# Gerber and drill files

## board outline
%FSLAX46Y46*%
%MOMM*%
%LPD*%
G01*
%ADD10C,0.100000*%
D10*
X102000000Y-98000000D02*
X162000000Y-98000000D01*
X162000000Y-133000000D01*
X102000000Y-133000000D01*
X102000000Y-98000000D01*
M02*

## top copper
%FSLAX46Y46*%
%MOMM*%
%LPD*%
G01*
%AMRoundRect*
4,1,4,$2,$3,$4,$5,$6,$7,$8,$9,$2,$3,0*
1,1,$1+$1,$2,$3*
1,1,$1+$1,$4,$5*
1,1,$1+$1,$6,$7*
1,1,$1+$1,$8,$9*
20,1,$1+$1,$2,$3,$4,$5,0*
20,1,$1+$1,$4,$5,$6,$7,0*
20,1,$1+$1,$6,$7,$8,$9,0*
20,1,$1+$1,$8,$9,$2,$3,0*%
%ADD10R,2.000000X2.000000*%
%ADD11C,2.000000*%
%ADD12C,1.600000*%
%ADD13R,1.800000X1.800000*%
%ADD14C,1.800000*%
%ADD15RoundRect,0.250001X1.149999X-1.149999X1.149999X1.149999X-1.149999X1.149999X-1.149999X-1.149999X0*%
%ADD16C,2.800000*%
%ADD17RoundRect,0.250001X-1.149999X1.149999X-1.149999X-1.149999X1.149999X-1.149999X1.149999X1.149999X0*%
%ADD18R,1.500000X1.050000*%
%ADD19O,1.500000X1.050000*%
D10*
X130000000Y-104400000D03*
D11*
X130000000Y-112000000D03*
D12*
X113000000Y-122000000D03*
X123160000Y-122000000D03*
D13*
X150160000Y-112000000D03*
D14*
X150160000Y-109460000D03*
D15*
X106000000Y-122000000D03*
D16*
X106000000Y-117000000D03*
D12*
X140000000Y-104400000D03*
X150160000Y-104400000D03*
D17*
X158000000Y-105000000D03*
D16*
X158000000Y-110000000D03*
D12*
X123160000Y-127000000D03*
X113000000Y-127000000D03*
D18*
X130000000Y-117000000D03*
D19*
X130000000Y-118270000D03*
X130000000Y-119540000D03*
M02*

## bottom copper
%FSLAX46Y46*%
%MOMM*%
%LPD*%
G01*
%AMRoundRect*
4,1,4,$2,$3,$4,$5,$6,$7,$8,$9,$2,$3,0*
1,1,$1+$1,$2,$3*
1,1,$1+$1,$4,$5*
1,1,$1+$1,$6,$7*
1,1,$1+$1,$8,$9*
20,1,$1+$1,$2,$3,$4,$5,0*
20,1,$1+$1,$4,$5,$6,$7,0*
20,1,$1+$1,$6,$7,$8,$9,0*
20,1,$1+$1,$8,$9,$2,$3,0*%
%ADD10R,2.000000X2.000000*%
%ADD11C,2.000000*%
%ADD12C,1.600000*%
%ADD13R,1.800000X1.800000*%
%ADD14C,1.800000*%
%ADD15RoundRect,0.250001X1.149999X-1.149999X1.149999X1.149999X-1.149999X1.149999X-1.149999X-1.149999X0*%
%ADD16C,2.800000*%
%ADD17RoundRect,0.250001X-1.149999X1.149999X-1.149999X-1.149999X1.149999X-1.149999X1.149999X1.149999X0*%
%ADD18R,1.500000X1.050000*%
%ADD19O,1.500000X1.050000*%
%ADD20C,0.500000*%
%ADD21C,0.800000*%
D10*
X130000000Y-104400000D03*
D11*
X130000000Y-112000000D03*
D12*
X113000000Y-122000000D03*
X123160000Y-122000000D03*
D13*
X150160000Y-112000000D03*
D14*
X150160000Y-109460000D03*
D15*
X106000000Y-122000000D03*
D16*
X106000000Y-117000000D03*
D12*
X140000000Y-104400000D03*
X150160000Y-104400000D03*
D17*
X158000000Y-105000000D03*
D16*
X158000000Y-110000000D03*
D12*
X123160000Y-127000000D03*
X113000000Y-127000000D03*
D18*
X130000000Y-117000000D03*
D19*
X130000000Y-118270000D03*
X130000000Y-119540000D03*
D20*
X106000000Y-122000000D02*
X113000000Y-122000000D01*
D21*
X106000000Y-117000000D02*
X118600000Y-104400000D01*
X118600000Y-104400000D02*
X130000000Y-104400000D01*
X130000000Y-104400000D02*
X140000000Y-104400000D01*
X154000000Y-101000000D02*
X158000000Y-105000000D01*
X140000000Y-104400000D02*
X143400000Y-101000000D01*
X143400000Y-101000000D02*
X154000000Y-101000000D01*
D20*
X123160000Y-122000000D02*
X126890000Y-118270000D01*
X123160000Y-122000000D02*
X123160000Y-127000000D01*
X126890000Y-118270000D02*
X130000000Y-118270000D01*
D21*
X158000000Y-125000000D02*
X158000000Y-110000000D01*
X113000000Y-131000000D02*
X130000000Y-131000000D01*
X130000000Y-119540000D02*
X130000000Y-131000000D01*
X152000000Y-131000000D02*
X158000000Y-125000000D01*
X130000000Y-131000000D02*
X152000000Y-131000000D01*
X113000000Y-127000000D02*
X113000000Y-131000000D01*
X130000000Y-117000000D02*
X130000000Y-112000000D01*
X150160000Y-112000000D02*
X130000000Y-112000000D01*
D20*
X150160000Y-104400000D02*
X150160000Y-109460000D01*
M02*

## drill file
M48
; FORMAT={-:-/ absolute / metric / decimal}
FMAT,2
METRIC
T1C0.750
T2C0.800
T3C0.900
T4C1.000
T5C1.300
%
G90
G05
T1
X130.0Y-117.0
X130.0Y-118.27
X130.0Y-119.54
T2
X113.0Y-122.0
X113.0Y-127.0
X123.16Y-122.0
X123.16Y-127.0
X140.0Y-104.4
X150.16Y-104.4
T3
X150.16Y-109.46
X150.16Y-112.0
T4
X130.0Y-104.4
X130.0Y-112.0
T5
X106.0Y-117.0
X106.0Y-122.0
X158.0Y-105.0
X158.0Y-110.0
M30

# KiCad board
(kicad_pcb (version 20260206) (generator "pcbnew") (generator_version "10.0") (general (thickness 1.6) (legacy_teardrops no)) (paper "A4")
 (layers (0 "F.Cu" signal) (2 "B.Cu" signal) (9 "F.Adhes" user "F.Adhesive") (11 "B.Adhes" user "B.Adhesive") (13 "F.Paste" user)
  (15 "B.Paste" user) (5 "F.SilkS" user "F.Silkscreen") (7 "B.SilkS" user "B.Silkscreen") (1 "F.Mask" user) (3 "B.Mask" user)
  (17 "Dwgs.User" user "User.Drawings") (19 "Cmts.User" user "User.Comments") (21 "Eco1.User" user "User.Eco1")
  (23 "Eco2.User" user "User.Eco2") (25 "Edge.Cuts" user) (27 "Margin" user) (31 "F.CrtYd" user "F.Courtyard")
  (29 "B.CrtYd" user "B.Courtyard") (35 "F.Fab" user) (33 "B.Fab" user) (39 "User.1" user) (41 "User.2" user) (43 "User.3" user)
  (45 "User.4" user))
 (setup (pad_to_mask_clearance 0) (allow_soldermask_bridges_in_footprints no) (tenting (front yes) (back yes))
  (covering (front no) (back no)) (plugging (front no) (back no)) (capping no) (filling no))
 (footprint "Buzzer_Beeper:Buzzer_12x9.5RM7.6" (layer "F.Cu") (at 130 104.4 -90)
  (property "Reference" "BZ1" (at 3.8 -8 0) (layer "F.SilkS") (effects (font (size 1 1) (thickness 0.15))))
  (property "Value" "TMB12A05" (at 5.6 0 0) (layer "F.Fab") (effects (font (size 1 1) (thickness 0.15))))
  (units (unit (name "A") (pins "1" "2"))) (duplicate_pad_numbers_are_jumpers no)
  (pad "1" thru_hole rect (at 0 0 270) (size 2 2) (drill 1) (layers "*.Cu" "*.Mask") (remove_unused_layers no) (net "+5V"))
  (pad "2" thru_hole circle (at 7.6 0 270) (size 2 2) (drill 1) (layers "*.Cu" "*.Mask") (remove_unused_layers no) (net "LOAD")))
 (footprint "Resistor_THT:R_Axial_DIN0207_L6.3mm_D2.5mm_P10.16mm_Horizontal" (layer "F.Cu") (at 113 122)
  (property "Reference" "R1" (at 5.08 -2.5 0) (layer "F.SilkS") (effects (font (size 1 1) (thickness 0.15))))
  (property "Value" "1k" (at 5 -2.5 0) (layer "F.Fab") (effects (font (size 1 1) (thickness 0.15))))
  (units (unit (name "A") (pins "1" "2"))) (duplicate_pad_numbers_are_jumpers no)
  (pad "1" thru_hole circle (at 0 0) (size 1.6 1.6) (drill 0.8) (layers "*.Cu" "*.Mask") (remove_unused_layers no) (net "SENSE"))
  (pad "2" thru_hole circle (at 10.16 0) (size 1.6 1.6) (drill 0.8) (layers "*.Cu" "*.Mask") (remove_unused_layers no) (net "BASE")))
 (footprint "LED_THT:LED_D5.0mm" (layer "F.Cu") (at 150.16 112 90)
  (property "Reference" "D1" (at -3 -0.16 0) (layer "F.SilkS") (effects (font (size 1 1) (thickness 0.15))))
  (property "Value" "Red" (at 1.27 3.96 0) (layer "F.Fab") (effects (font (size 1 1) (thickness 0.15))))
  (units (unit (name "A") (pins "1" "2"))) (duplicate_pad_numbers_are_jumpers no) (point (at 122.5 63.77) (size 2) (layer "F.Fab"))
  (pad "1" thru_hole rect (at 0 0 90) (size 1.8 1.8) (drill 0.9) (layers "*.Cu" "*.Mask") (remove_unused_layers no) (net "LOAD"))
  (pad "2" thru_hole circle (at 2.54 0 90) (size 1.8 1.8) (drill 0.9) (layers "*.Cu" "*.Mask") (remove_unused_layers no) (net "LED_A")))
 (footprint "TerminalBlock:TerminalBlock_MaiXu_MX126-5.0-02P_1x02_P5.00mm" (layer "F.Cu") (at 106 122 90)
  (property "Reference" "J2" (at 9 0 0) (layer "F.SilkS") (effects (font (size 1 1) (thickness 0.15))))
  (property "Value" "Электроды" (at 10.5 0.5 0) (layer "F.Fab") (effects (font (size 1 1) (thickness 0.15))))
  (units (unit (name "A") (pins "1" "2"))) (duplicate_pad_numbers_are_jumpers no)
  (pad "1" thru_hole roundrect (at 0 0 90) (size 2.8 2.8) (drill 1.3) (layers "*.Cu" "*.Mask") (remove_unused_layers no)
   (roundrect_rratio 0.089286) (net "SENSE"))
  (pad "2" thru_hole circle (at 5 0 90) (size 2.8 2.8) (drill 1.3) (layers "*.Cu" "*.Mask") (remove_unused_layers no) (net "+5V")))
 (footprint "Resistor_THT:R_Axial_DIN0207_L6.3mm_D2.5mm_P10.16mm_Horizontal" (layer "F.Cu") (at 140 104.4)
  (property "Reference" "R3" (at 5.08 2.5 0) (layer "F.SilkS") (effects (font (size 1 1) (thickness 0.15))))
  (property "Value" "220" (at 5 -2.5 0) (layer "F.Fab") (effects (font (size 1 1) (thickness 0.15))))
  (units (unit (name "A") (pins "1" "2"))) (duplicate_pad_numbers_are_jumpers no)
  (pad "1" thru_hole circle (at 0 0) (size 1.6 1.6) (drill 0.8) (layers "*.Cu" "*.Mask") (remove_unused_layers no) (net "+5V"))
  (pad "2" thru_hole circle (at 10.16 0) (size 1.6 1.6) (drill 0.8) (layers "*.Cu" "*.Mask") (remove_unused_layers no) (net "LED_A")))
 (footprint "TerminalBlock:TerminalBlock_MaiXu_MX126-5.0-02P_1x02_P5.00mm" (layer "F.Cu") (at 158 105 -90)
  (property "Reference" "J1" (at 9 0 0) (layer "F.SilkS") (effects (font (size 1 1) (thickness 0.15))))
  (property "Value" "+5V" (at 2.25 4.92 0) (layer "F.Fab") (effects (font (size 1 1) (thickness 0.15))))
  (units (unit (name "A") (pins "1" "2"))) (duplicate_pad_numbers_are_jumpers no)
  (pad "1" thru_hole roundrect (at 0 0 270) (size 2.8 2.8) (drill 1.3) (layers "*.Cu" "*.Mask") (remove_unused_layers no)
   (roundrect_rratio 0.089286) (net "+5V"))
  (pad "2" thru_hole circle (at 5 0 270) (size 2.8 2.8) (drill 1.3) (layers "*.Cu" "*.Mask") (remove_unused_layers no) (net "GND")))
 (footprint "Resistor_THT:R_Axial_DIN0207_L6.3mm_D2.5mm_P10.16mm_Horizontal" (layer "F.Cu") (at 123.16 127 180)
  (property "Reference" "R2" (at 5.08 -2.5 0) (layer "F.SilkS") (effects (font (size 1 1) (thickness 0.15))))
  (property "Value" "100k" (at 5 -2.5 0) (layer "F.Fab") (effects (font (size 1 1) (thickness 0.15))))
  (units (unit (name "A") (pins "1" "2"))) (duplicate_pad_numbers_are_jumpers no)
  (pad "1" thru_hole circle (at 0 0 180) (size 1.6 1.6) (drill 0.8) (layers "*.Cu" "*.Mask") (remove_unused_layers no) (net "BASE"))
  (pad "2" thru_hole circle (at 10.16 0 180) (size 1.6 1.6) (drill 0.8) (layers "*.Cu" "*.Mask") (remove_unused_layers no) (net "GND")))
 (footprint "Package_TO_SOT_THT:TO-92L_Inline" (layer "F.Cu") (at 130 117 -90)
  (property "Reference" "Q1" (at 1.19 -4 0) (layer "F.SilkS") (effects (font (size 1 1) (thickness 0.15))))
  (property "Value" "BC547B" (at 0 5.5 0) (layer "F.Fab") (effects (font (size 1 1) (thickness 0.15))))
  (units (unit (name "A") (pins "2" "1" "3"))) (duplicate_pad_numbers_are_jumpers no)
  (pad "1" thru_hole rect (at 0 0 270) (size 1.05 1.5) (drill 0.75) (layers "*.Cu" "*.Mask") (remove_unused_layers no) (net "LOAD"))
  (pad "2" thru_hole oval (at 1.27 0 270) (size 1.05 1.5) (drill 0.75) (layers "*.Cu" "*.Mask") (remove_unused_layers no) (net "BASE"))
  (pad "3" thru_hole oval (at 2.54 0 270) (size 1.05 1.5) (drill 0.75) (layers "*.Cu" "*.Mask") (remove_unused_layers no) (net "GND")))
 (gr_rect (start 102 98) (end 162 133) (stroke (width 0.1) (type default)) (fill no) (layer "Edge.Cuts"))
 (segment (start 106 122) (end 113 122) (width 0.5) (layer "B.Cu") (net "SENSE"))
 (segment (start 106 117) (end 118.6 104.4) (width 0.8) (layer "B.Cu") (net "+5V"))
 (segment (start 118.6 104.4) (end 130 104.4) (width 0.8) (layer "B.Cu") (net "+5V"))
 (segment (start 130 104.4) (end 140 104.4) (width 0.8) (layer "B.Cu") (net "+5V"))
 (segment (start 154 101) (end 158 105) (width 0.8) (layer "B.Cu") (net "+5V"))
 (segment (start 140 104.4) (end 143.4 101) (width 0.8) (layer "B.Cu") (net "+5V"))
 (segment (start 143.4 101) (end 154 101) (width 0.8) (layer "B.Cu") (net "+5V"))
 (segment (start 123.16 122) (end 126.89 118.27) (width 0.5) (layer "B.Cu") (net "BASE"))
 (segment (start 123.16 122) (end 123.16 127) (width 0.5) (layer "B.Cu") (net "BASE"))
 (segment (start 126.89 118.27) (end 130 118.27) (width 0.5) (layer "B.Cu") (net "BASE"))
 (segment (start 158 125) (end 158 110) (width 0.8) (layer "B.Cu") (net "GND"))
 (segment (start 113 131) (end 130 131) (width 0.8) (layer "B.Cu") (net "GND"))
 (segment (start 130 119.54) (end 130 131) (width 0.8) (layer "B.Cu") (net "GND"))
 (segment (start 152 131) (end 158 125) (width 0.8) (layer "B.Cu") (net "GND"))
 (segment (start 130 131) (end 152 131) (width 0.8) (layer "B.Cu") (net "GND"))
 (segment (start 113 127) (end 113 131) (width 0.8) (layer "B.Cu") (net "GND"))
 (segment (start 130 117) (end 130 112) (width 0.8) (layer "B.Cu") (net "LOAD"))
 (segment (start 150.16 112) (end 130 112) (width 0.8) (layer "B.Cu") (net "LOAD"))
 (segment (start 150.16 104.4) (end 150.16 109.46) (width 0.5) (layer "B.Cu") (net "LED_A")))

